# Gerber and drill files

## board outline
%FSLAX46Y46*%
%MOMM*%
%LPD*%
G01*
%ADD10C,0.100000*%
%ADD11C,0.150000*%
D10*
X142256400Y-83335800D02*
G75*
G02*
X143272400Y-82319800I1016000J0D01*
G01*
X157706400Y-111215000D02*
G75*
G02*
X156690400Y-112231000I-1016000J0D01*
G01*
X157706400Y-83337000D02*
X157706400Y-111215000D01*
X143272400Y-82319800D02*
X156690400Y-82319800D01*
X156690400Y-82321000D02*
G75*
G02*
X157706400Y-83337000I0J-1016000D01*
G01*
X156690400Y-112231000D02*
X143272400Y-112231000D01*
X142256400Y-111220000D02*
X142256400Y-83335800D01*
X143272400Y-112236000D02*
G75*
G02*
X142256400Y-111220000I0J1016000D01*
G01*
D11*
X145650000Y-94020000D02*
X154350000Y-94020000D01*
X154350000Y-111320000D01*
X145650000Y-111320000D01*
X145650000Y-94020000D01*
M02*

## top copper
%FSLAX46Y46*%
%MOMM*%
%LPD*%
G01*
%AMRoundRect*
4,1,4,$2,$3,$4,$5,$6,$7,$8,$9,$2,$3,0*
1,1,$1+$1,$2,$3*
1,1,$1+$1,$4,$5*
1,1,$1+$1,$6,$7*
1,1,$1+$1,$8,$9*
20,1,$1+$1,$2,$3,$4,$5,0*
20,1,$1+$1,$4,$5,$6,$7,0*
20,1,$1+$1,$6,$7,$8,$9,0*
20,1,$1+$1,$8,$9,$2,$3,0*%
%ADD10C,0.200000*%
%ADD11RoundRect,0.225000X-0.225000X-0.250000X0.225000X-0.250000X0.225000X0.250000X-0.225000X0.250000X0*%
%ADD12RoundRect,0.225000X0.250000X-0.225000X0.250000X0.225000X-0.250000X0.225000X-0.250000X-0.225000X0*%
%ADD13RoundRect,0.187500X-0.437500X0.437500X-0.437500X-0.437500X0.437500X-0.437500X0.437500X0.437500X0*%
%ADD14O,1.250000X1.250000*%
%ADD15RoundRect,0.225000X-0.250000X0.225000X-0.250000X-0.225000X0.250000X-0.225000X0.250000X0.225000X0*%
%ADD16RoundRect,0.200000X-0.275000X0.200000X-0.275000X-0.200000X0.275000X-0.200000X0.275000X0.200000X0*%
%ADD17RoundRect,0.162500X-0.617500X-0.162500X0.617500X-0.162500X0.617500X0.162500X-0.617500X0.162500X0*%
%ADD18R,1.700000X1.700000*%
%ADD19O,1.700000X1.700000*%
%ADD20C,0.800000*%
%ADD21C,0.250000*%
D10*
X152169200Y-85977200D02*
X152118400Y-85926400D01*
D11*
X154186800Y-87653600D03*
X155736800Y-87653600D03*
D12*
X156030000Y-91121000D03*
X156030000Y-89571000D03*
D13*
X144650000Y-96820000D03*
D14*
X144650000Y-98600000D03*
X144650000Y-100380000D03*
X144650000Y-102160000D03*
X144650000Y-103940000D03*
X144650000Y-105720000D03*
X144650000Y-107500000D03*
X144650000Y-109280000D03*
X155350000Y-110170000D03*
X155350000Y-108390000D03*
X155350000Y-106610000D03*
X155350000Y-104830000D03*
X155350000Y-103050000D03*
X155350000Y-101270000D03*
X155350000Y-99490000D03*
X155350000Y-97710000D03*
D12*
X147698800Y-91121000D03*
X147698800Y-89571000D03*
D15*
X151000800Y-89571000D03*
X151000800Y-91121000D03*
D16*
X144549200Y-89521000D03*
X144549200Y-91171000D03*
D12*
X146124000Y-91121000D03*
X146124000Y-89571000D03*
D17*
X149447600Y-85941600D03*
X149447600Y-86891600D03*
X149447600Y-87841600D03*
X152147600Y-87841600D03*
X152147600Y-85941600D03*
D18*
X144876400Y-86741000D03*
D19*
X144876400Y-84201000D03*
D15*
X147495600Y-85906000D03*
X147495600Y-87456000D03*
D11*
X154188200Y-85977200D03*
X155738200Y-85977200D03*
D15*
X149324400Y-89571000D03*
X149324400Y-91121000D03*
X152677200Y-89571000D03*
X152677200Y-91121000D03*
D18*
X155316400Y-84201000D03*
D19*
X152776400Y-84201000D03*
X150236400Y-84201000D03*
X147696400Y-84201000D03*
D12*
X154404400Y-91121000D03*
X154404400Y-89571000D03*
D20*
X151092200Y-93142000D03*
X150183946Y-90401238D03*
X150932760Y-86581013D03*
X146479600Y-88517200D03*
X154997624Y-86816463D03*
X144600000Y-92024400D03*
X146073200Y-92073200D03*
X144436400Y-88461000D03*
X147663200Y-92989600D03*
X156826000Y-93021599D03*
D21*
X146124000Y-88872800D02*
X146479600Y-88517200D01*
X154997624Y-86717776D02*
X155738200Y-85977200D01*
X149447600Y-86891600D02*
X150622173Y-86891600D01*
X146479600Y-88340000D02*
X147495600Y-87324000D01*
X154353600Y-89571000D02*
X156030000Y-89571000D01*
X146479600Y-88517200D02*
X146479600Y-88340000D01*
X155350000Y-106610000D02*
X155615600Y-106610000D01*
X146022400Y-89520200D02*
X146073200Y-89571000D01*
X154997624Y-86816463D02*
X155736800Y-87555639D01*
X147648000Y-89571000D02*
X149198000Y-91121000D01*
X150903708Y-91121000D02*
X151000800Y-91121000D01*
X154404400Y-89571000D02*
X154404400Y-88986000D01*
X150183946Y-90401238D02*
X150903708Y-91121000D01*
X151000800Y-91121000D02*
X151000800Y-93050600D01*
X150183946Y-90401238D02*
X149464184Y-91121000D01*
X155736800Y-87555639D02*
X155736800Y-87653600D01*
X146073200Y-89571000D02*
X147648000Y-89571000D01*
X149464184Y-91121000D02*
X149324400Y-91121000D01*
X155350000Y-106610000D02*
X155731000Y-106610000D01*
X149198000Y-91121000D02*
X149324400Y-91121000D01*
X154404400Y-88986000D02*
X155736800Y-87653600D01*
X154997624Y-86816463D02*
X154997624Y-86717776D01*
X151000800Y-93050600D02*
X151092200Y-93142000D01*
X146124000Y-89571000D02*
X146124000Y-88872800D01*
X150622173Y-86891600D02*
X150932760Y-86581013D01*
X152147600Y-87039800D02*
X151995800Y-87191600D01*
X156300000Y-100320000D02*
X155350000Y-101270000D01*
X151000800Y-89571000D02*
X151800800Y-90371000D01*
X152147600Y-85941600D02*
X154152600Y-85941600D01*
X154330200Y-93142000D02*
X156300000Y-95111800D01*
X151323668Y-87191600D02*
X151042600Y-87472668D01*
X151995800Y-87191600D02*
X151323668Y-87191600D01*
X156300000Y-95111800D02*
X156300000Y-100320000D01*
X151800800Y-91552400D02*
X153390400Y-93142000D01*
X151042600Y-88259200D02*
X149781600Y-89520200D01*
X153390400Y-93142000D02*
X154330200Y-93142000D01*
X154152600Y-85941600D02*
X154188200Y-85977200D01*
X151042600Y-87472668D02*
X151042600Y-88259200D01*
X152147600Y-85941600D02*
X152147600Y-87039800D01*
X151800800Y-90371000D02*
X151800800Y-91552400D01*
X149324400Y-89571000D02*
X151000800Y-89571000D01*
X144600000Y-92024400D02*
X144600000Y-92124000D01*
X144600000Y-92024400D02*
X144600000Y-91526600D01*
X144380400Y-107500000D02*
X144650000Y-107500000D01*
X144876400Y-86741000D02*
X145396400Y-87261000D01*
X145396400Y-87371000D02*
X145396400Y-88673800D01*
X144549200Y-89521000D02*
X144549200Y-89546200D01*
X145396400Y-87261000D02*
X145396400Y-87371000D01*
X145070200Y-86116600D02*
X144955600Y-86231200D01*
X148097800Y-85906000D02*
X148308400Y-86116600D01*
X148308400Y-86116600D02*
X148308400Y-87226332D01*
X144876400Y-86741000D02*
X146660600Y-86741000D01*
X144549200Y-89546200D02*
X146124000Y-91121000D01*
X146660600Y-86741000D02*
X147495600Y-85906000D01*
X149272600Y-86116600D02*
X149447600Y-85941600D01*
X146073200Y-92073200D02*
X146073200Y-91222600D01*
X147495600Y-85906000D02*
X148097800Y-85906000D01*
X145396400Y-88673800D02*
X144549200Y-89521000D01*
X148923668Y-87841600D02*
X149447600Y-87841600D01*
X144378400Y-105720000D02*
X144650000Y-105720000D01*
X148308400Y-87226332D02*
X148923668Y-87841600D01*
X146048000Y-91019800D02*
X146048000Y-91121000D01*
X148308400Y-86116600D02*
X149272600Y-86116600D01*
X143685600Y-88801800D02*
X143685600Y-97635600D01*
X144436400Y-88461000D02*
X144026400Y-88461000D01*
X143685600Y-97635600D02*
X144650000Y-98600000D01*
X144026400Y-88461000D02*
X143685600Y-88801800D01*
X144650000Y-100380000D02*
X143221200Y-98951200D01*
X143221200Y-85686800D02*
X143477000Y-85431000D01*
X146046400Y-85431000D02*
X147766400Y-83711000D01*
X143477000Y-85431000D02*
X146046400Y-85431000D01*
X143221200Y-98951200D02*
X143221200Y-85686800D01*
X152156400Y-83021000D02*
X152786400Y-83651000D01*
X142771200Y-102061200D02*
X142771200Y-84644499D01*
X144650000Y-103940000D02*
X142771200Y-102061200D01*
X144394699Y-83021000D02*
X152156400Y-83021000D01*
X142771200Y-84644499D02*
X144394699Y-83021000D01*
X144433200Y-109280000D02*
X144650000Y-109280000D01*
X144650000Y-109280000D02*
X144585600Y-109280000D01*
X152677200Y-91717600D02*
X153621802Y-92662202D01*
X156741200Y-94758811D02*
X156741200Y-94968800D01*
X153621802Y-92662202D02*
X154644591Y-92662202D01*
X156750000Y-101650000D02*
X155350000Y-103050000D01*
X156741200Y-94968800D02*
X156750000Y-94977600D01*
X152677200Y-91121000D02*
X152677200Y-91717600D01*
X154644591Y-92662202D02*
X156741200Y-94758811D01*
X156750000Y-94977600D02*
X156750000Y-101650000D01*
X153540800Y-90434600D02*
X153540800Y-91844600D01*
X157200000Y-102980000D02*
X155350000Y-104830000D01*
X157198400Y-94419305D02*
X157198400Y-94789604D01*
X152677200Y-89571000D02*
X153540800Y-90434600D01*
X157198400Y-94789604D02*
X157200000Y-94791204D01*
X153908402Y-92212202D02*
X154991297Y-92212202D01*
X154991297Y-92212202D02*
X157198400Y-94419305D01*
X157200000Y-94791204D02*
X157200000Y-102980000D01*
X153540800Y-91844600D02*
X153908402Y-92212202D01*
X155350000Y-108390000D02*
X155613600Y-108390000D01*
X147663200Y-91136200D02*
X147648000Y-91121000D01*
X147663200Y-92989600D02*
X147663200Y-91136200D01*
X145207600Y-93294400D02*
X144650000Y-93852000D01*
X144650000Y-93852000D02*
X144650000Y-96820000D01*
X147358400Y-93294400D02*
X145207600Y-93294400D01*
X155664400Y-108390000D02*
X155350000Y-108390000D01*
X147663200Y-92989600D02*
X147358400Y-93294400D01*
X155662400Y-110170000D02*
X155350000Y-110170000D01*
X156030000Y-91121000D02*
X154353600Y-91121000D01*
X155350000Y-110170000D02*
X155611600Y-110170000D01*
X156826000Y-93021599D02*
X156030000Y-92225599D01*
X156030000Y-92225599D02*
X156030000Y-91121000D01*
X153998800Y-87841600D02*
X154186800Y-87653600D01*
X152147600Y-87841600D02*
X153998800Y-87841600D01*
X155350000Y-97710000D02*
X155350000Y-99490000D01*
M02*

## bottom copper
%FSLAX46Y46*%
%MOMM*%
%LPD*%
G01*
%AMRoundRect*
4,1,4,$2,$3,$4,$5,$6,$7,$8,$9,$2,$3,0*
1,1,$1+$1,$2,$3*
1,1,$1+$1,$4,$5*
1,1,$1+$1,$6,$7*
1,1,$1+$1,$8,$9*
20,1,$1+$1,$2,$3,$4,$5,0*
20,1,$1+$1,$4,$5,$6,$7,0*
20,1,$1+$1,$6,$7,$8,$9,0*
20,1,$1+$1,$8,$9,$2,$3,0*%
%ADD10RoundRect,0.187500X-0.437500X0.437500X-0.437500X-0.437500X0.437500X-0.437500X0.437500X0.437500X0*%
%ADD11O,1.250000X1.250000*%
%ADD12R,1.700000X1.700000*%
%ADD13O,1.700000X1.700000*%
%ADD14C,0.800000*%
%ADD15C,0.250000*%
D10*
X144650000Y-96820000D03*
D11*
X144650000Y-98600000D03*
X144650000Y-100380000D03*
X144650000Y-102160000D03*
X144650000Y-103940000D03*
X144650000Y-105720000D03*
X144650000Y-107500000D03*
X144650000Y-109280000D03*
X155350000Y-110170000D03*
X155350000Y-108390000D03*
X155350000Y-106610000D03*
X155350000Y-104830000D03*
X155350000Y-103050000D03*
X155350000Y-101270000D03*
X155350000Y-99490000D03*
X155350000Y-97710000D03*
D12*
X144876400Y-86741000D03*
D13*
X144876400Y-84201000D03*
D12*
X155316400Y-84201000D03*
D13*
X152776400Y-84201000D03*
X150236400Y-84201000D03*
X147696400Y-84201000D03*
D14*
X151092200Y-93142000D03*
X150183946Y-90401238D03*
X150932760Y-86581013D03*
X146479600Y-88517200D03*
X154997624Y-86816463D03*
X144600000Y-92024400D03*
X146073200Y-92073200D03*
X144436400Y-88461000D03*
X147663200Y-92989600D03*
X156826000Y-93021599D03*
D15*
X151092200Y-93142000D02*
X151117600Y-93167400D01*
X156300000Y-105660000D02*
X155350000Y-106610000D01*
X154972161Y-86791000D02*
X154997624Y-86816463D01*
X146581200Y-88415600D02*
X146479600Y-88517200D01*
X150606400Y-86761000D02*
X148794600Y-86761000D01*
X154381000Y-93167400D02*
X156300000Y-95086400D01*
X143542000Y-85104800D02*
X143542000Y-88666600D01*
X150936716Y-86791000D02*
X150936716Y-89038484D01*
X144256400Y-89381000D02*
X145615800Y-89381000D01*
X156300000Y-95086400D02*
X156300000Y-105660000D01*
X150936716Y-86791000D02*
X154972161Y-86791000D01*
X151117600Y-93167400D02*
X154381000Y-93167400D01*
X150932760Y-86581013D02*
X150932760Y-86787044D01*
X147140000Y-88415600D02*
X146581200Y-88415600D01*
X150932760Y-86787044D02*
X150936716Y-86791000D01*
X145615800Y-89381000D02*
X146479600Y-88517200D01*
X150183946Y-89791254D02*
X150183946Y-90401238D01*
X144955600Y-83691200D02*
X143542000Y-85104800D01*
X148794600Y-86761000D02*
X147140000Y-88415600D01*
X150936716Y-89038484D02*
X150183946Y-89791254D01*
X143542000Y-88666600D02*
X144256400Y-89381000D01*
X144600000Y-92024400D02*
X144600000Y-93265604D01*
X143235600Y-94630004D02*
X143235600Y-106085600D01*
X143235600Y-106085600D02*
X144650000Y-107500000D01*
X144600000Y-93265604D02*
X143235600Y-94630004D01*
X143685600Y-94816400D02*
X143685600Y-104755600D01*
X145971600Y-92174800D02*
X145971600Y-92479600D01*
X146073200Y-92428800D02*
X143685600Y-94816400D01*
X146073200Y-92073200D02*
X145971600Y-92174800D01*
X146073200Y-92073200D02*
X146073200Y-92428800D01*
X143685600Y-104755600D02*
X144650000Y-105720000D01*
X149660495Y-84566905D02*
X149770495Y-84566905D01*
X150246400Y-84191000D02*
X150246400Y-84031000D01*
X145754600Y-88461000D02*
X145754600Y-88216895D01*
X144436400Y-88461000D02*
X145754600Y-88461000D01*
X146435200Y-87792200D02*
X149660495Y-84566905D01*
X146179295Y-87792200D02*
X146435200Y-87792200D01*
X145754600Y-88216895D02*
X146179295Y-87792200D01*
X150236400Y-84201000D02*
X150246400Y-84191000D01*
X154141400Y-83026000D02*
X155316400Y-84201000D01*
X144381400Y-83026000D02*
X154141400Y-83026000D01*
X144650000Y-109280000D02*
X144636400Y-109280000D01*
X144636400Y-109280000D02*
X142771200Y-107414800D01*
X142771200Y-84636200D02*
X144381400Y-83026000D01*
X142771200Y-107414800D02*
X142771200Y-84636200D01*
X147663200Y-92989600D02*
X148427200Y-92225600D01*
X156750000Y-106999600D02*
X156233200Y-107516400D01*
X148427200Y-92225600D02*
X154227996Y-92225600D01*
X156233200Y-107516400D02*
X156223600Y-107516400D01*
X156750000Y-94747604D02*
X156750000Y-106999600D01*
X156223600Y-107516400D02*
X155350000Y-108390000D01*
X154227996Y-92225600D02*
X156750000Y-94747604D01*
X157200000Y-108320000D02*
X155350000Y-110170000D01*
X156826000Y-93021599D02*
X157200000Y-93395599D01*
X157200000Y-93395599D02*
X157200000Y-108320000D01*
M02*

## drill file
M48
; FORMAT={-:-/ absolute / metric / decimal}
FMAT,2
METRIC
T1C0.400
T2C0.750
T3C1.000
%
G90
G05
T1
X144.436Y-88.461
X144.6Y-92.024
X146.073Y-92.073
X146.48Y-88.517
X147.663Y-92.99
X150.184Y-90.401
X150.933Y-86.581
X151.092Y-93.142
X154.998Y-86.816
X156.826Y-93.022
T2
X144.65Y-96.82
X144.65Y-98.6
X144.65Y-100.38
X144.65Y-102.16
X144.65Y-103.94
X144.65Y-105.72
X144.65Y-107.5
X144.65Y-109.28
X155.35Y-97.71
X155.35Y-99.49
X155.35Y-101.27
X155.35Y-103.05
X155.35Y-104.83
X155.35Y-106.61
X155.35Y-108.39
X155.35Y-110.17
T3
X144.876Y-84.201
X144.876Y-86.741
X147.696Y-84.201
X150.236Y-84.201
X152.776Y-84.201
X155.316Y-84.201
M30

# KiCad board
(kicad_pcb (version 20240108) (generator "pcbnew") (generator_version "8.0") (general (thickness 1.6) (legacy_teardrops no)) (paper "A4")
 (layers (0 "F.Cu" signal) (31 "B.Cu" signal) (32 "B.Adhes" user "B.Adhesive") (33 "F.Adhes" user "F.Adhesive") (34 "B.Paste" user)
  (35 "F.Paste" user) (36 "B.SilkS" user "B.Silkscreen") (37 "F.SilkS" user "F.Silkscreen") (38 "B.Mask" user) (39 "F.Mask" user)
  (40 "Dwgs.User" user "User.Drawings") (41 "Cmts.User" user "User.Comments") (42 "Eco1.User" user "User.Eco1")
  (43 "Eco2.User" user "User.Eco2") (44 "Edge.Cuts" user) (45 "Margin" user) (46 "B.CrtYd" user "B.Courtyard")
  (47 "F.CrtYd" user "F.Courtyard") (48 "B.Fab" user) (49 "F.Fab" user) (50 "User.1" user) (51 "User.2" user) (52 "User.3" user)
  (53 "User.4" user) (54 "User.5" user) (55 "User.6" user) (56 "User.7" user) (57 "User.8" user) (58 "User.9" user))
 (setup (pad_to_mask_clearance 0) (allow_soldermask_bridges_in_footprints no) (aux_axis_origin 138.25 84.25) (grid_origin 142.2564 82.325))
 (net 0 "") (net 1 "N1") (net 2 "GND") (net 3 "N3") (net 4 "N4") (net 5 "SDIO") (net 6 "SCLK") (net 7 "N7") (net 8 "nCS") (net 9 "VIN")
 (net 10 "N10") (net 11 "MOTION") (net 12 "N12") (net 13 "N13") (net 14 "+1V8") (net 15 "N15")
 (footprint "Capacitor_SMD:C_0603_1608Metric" (layer "F.Cu") (at 154.9618 87.6536)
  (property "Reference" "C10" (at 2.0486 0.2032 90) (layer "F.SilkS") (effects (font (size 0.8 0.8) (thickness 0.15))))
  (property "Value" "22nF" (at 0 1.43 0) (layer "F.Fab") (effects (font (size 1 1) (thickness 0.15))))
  (pad "1" smd roundrect (at -0.775 0) (size 0.9 0.95) (layers "F.Cu" "F.Paste" "F.Mask") (roundrect_rratio 0.25) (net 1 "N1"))
  (pad "2" smd roundrect (at 0.775 0) (size 0.9 0.95) (layers "F.Cu" "F.Paste" "F.Mask") (roundrect_rratio 0.25) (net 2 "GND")))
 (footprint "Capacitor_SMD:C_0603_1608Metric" (layer "F.Cu") (at 156.03 90.346 90)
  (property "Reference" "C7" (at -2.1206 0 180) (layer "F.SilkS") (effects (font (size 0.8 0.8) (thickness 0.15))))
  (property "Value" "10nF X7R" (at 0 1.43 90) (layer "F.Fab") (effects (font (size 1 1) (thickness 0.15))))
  (pad "1" smd roundrect (at -0.775 0 90) (size 0.9 0.95) (layers "F.Cu" "F.Paste" "F.Mask") (roundrect_rratio 0.25) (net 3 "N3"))
  (pad "2" smd roundrect (at 0.775 0 90) (size 0.9 0.95) (layers "F.Cu" "F.Paste" "F.Mask") (roundrect_rratio 0.25) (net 2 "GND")))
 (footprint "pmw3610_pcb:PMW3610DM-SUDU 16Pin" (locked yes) (layer "F.Cu") (at 150 102.988 90)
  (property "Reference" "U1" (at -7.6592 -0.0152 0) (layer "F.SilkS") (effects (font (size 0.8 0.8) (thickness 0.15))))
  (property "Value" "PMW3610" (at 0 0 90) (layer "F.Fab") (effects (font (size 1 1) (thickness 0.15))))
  (fp_rect (start 8.968 -4.35) (end -8.332 4.35) (stroke (width 0.15) (type solid)) (fill none) (layer "Edge.Cuts"))
  (pad "1" thru_hole roundrect (at 6.168 -5.35 270) (size 1.25 1.25) (drill 0.75) (layers "*.Cu" "*.Mask") (remove_unused_layers no)
   (roundrect_rratio 0.15) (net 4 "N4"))
  (pad "2" thru_hole oval (at 4.388 -5.35 270) (size 1.25 1.25) (drill 0.75) (layers "*.Cu" "*.Mask") (remove_unused_layers no)
   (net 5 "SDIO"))
  (pad "3" thru_hole oval (at 2.608 -5.35 270) (size 1.25 1.25) (drill 0.75) (layers "*.Cu" "*.Mask") (remove_unused_layers no)
   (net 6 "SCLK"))
  (pad "4" thru_hole oval (at 0.828 -5.35 270) (size 1.25 1.25) (drill 0.75) (layers "*.Cu" "*.Mask") (remove_unused_layers no) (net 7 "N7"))
  (pad "5" thru_hole oval (at -0.952 -5.35 270) (size 1.25 1.25) (drill 0.75) (layers "*.Cu" "*.Mask") (remove_unused_layers no)
   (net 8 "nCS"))
  (pad "6" thru_hole oval (at -2.732 -5.35 270) (size 1.25 1.25) (drill 0.75) (layers "*.Cu" "*.Mask") (remove_unused_layers no)
   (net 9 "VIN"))
  (pad "7" thru_hole oval (at -4.512 -5.35 270) (size 1.25 1.25) (drill 0.75) (layers "*.Cu" "*.Mask") (remove_unused_layers no)
   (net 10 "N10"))
  (pad "8" thru_hole oval (at -6.292 -5.35 270) (size 1.25 1.25) (drill 0.75) (layers "*.Cu" "*.Mask") (remove_unused_layers no)
   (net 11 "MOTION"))
  (pad "9" thru_hole oval (at -7.182 5.35 270) (size 1.25 1.25) (drill 0.75) (layers "*.Cu" "*.Mask") (remove_unused_layers no) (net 3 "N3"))
  (pad "10" thru_hole oval (at -5.402 5.35 270) (size 1.25 1.25) (drill 0.75) (layers "*.Cu" "*.Mask") (remove_unused_layers no)
   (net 4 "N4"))
  (pad "11" thru_hole oval (at -3.622 5.35 270) (size 1.25 1.25) (drill 0.75) (layers "*.Cu" "*.Mask") (remove_unused_layers no)
   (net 2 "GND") (thermal_bridge_angle 45))
  (pad "12" thru_hole oval (at -1.842 5.35 270) (size 1.25 1.25) (drill 0.75) (layers "*.Cu" "*.Mask") (remove_unused_layers no)
   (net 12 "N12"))
  (pad "13" thru_hole oval (at -0.062 5.35 270) (size 1.25 1.25) (drill 0.75) (layers "*.Cu" "*.Mask") (remove_unused_layers no)
   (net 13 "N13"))
  (pad "14" thru_hole oval (at 1.718 5.35 270) (size 1.25 1.25) (drill 0.75) (layers "*.Cu" "*.Mask") (remove_unused_layers no)
   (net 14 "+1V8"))
  (pad "15" thru_hole oval (at 3.498 5.35 270) (size 1.25 1.25) (drill 0.75) (layers "*.Cu" "*.Mask") (remove_unused_layers no)
   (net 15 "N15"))
  (pad "16" thru_hole oval (at 5.278 5.35 270) (size 1.25 1.25) (drill 0.75) (layers "*.Cu" "*.Mask") (remove_unused_layers no)
   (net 15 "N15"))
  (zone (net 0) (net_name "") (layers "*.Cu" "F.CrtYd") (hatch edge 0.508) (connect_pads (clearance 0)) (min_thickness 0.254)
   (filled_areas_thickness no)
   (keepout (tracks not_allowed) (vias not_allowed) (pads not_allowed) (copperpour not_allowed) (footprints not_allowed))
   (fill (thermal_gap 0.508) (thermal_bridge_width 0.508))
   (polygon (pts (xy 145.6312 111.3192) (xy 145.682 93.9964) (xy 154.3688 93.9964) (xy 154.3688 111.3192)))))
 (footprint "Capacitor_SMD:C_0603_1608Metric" (layer "F.Cu") (at 147.6988 90.346 90)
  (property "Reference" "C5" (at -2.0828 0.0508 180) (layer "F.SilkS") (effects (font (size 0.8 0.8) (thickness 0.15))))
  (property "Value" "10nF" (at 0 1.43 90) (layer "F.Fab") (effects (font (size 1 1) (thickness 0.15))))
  (pad "1" smd roundrect (at -0.775 0 90) (size 0.9 0.95) (layers "F.Cu" "F.Paste" "F.Mask") (roundrect_rratio 0.25) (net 4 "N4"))
  (pad "2" smd roundrect (at 0.775 0 90) (size 0.9 0.95) (layers "F.Cu" "F.Paste" "F.Mask") (roundrect_rratio 0.25) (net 2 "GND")))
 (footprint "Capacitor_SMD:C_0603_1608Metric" (layer "F.Cu") (at 151.0008 90.346 -90)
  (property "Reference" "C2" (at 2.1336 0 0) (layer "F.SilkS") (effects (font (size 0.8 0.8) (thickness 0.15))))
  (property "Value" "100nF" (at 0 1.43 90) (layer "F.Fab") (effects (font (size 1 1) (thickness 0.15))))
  (pad "1" smd roundrect (at -0.775 0 270) (size 0.9 0.95) (layers "F.Cu" "F.Paste" "F.Mask") (roundrect_rratio 0.25) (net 14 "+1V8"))
  (pad "2" smd roundrect (at 0.775 0 270) (size 0.9 0.95) (layers "F.Cu" "F.Paste" "F.Mask") (roundrect_rratio 0.25) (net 2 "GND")))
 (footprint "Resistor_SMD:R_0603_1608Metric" (layer "F.Cu") (at 144.5492 90.346 -90)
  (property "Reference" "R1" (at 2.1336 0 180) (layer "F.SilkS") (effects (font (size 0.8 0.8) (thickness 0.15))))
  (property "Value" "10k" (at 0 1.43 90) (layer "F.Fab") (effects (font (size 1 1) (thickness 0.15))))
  (pad "1" smd roundrect (at -0.825 0 270) (size 0.8 0.95) (layers "F.Cu" "F.Paste" "F.Mask") (roundrect_rratio 0.25) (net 9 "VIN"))
  (pad "2" smd roundrect (at 0.825 0 270) (size 0.8 0.95) (layers "F.Cu" "F.Paste" "F.Mask") (roundrect_rratio 0.25) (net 10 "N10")))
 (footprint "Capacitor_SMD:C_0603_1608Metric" (layer "F.Cu") (at 146.124 90.346 90)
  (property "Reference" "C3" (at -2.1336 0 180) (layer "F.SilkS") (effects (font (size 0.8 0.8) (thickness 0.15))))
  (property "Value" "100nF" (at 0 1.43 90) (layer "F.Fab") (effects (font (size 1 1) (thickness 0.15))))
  (pad "1" smd roundrect (at -0.775 0 90) (size 0.9 0.95) (layers "F.Cu" "F.Paste" "F.Mask") (roundrect_rratio 0.25) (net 9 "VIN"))
  (pad "2" smd roundrect (at 0.775 0 90) (size 0.9 0.95) (layers "F.Cu" "F.Paste" "F.Mask") (roundrect_rratio 0.25) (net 2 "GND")))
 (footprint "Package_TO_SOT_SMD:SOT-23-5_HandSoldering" (layer "F.Cu") (at 150.7976 86.8916)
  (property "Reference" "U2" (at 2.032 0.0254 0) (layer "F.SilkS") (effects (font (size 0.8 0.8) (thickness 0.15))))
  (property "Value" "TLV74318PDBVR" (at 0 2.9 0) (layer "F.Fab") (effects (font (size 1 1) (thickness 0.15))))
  (pad "1" smd roundrect (at -1.35 -0.95) (size 1.56 0.65) (layers "F.Cu" "F.Paste" "F.Mask") (roundrect_rratio 0.25) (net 9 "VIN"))
  (pad "2" smd roundrect (at -1.35 0) (size 1.56 0.65) (layers "F.Cu" "F.Paste" "F.Mask") (roundrect_rratio 0.25) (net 2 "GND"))
  (pad "3" smd roundrect (at -1.35 0.95) (size 1.56 0.65) (layers "F.Cu" "F.Paste" "F.Mask") (roundrect_rratio 0.25) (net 9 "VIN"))
  (pad "4" smd roundrect (at 1.35 0.95) (size 1.56 0.65) (layers "F.Cu" "F.Paste" "F.Mask") (roundrect_rratio 0.25) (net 1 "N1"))
  (pad "5" smd roundrect (at 1.35 -0.95) (size 1.56 0.65) (layers "F.Cu" "F.Paste" "F.Mask") (roundrect_rratio 0.25) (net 14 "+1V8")))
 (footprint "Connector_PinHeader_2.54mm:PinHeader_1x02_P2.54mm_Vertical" (layer "F.Cu") (at 144.8764 86.741 180)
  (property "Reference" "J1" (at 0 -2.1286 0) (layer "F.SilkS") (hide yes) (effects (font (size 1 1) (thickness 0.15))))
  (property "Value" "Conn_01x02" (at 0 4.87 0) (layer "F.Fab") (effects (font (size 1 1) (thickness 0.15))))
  (pad "1" thru_hole rect (at 0 0 180) (size 1.7 1.7) (drill 1) (layers "*.Cu" "*.Mask") (remove_unused_layers no) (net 9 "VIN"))
  (pad "2" thru_hole oval (at 0 2.54 180) (size 1.7 1.7) (drill 1) (layers "*.Cu" "*.Mask") (remove_unused_layers no) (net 2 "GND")))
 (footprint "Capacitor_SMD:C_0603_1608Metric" (layer "F.Cu") (at 147.4956 86.681 -90)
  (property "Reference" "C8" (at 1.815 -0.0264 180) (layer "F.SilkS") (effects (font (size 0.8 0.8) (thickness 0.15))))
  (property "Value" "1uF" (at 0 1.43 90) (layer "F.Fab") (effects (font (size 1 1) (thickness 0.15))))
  (pad "1" smd roundrect (at -0.775 0 270) (size 0.9 0.95) (layers "F.Cu" "F.Paste" "F.Mask") (roundrect_rratio 0.25) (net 9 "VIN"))
  (pad "2" smd roundrect (at 0.775 0 270) (size 0.9 0.95) (layers "F.Cu" "F.Paste" "F.Mask") (roundrect_rratio 0.25) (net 2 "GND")))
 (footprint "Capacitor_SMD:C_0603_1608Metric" (layer "F.Cu") (at 154.9632 85.9772)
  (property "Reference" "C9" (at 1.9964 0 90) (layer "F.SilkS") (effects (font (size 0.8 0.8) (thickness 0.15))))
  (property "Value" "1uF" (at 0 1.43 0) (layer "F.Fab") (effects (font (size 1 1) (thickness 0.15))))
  (pad "1" smd roundrect (at -0.775 0) (size 0.9 0.95) (layers "F.Cu" "F.Paste" "F.Mask") (roundrect_rratio 0.25) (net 14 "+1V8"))
  (pad "2" smd roundrect (at 0.775 0) (size 0.9 0.95) (layers "F.Cu" "F.Paste" "F.Mask") (roundrect_rratio 0.25) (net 2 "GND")))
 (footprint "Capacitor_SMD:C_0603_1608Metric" (layer "F.Cu") (at 149.3244 90.346 -90)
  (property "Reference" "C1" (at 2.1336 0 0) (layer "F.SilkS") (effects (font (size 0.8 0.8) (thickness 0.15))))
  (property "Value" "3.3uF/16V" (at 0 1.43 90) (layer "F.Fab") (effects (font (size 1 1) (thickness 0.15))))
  (pad "1" smd roundrect (at -0.775 0 270) (size 0.9 0.95) (layers "F.Cu" "F.Paste" "F.Mask") (roundrect_rratio 0.25) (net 14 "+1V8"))
  (pad "2" smd roundrect (at 0.775 0 270) (size 0.9 0.95) (layers "F.Cu" "F.Paste" "F.Mask") (roundrect_rratio 0.25) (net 2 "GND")))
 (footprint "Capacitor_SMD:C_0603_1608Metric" (layer "F.Cu") (at 152.6772 90.346 -90)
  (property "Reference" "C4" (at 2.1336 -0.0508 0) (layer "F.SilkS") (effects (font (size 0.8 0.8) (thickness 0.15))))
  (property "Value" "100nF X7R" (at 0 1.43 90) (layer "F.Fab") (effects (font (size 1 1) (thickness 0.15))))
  (pad "1" smd roundrect (at -0.775 0 270) (size 0.9 0.95) (layers "F.Cu" "F.Paste" "F.Mask") (roundrect_rratio 0.25) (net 12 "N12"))
  (pad "2" smd roundrect (at 0.775 0 270) (size 0.9 0.95) (layers "F.Cu" "F.Paste" "F.Mask") (roundrect_rratio 0.25) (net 13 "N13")))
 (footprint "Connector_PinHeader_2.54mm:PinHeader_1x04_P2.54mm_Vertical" (layer "F.Cu") (at 155.3164 84.201 -90)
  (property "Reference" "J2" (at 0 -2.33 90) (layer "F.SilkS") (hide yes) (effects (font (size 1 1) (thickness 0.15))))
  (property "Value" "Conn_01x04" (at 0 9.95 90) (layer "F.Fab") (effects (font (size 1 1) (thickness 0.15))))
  (pad "1" thru_hole rect (at 0 0 270) (size 1.7 1.7) (drill 1) (layers "*.Cu" "*.Mask") (remove_unused_layers no) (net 11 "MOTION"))
  (pad "2" thru_hole oval (at 0 2.54 270) (size 1.7 1.7) (drill 1) (layers "*.Cu" "*.Mask") (remove_unused_layers no) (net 8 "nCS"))
  (pad "3" thru_hole oval (at 0 5.08 270) (size 1.7 1.7) (drill 1) (layers "*.Cu" "*.Mask") (remove_unused_layers no) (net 5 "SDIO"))
  (pad "4" thru_hole oval (at 0 7.62 270) (size 1.7 1.7) (drill 1) (layers "*.Cu" "*.Mask") (remove_unused_layers no) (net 6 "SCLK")))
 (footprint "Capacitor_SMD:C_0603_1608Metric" (layer "F.Cu") (at 154.4044 90.346 90)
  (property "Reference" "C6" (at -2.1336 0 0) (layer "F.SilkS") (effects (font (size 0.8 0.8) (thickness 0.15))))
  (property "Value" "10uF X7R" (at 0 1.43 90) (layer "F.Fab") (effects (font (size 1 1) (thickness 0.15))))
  (pad "1" smd roundrect (at -0.775 0 90) (size 0.9 0.95) (layers "F.Cu" "F.Paste" "F.Mask") (roundrect_rratio 0.25) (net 3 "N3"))
  (pad "2" smd roundrect (at 0.775 0 90) (size 0.9 0.95) (layers "F.Cu" "F.Paste" "F.Mask") (roundrect_rratio 0.25) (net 2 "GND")))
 (gr_line (start 152.1692 85.9772) (end 152.1184 85.9264) (stroke (width 0.2) (type default)) (layer "F.Cu") (net 14))
 (gr_arc (start 142.2564 83.3358) (mid 142.55398 82.61738) (end 143.2724 82.3198) (stroke (width 0.1) (type default)) (layer "Edge.Cuts"))
 (gr_arc (start 157.7064 111.215) (mid 157.40882 111.93342) (end 156.6904 112.231) (stroke (width 0.1) (type default)) (layer "Edge.Cuts"))
 (gr_line (start 157.7064 83.337) (end 157.7064 111.215) (stroke (width 0.1) (type default)) (layer "Edge.Cuts"))
 (gr_line (start 143.2724 82.3198) (end 156.6904 82.3198) (stroke (width 0.1) (type default)) (layer "Edge.Cuts"))
 (gr_arc (start 156.6904 82.321) (mid 157.40882 82.61858) (end 157.7064 83.337) (stroke (width 0.1) (type default)) (layer "Edge.Cuts"))
 (gr_line (start 156.6904 112.231) (end 143.2724 112.231) (stroke (width 0.1) (type default)) (layer "Edge.Cuts"))
 (gr_line (start 142.2564 111.22) (end 142.2564 83.3358) (stroke (width 0.1) (type default)) (layer "Edge.Cuts"))
 (gr_arc (start 143.2724 112.236) (mid 142.55398 111.93842) (end 142.2564 111.22) (stroke (width 0.1) (type default)) (layer "Edge.Cuts"))
 (segment (start 146.124 88.8728) (end 146.4796 88.5172) (width 0.25) (layer "F.Cu") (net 2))
 (segment (start 154.997624 86.717776) (end 155.7382 85.9772) (width 0.25) (layer "F.Cu") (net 2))
 (segment (start 149.4476 86.8916) (end 150.622173 86.8916) (width 0.25) (layer "F.Cu") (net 2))
 (segment (start 146.4796 88.34) (end 147.4956 87.324) (width 0.25) (layer "F.Cu") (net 2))
 (segment (start 154.3536 89.571) (end 156.03 89.571) (width 0.25) (layer "F.Cu") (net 2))
 (segment (start 146.4796 88.5172) (end 146.4796 88.34) (width 0.25) (layer "F.Cu") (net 2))
 (segment (start 155.35 106.61) (end 155.6156 106.61) (width 0.25) (layer "F.Cu") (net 2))
 (segment (start 146.0224 89.5202) (end 146.0732 89.571) (width 0.25) (layer "F.Cu") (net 2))
 (segment (start 154.997624 86.816463) (end 155.7368 87.555639) (width 0.25) (layer "F.Cu") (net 2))
 (segment (start 147.648 89.571) (end 149.198 91.121) (width 0.25) (layer "F.Cu") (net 2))
 (segment (start 150.903708 91.121) (end 151.0008 91.121) (width 0.25) (layer "F.Cu") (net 2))
 (segment (start 154.4044 89.571) (end 154.4044 88.986) (width 0.25) (layer "F.Cu") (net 2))
 (segment (start 150.183946 90.401238) (end 150.903708 91.121) (width 0.25) (layer "F.Cu") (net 2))
 (segment (start 151.0008 91.121) (end 151.0008 93.0506) (width 0.25) (layer "F.Cu") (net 2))
 (segment (start 150.183946 90.401238) (end 149.464184 91.121) (width 0.25) (layer "F.Cu") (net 2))
 (segment (start 155.7368 87.555639) (end 155.7368 87.6536) (width 0.25) (layer "F.Cu") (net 2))
 (segment (start 146.0732 89.571) (end 147.648 89.571) (width 0.25) (layer "F.Cu") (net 2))
 (segment (start 149.464184 91.121) (end 149.3244 91.121) (width 0.25) (layer "F.Cu") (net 2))
 (segment (start 155.35 106.61) (end 155.731 106.61) (width 0.25) (layer "F.Cu") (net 2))
 (segment (start 149.198 91.121) (end 149.3244 91.121) (width 0.25) (layer "F.Cu") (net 2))
 (segment (start 154.4044 88.986) (end 155.7368 87.6536) (width 0.25) (layer "F.Cu") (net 2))
 (segment (start 154.997624 86.816463) (end 154.997624 86.717776) (width 0.25) (layer "F.Cu") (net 2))
 (segment (start 151.0008 93.0506) (end 151.0922 93.142) (width 0.25) (layer "F.Cu") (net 2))
 (segment (start 146.124 89.571) (end 146.124 88.8728) (width 0.25) (layer "F.Cu") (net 2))
 (segment (start 150.622173 86.8916) (end 150.93276 86.581013) (width 0.25) (layer "F.Cu") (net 2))
 (via (at 151.0922 93.142) (size 0.8) (drill 0.4) (layers "F.Cu" "B.Cu") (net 2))
 (via (at 150.183946 90.401238) (size 0.8) (drill 0.4) (layers "F.Cu" "B.Cu") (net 2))
 (via (at 150.93276 86.581013) (size 0.8) (drill 0.4) (layers "F.Cu" "B.Cu") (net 2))
 (via (at 146.4796 88.5172) (size 0.8) (drill 0.4) (layers "F.Cu" "B.Cu") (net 2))
 (via (at 154.997624 86.816463) (size 0.8) (drill 0.4) (layers "F.Cu" "B.Cu") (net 2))
 (segment (start 151.0922 93.142) (end 151.1176 93.1674) (width 0.25) (layer "B.Cu") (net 2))
 (segment (start 156.3 105.66) (end 155.35 106.61) (width 0.25) (layer "B.Cu") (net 2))
 (segment (start 154.972161 86.791) (end 154.997624 86.816463) (width 0.25) (layer "B.Cu") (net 2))
 (segment (start 146.5812 88.4156) (end 146.4796 88.5172) (width 0.25) (layer "B.Cu") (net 2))
 (segment (start 150.6064 86.761) (end 148.7946 86.761) (width 0.25) (layer "B.Cu") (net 2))
 (segment (start 154.381 93.1674) (end 156.3 95.0864) (width 0.25) (layer "B.Cu") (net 2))
 (segment (start 143.542 85.1048) (end 143.542 88.6666) (width 0.25) (layer "B.Cu") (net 2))
 (segment (start 150.936716 86.791) (end 150.936716 89.038484) (width 0.25) (layer "B.Cu") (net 2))
 (segment (start 144.2564 89.381) (end 145.6158 89.381) (width 0.25) (layer "B.Cu") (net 2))
 (segment (start 156.3 95.0864) (end 156.3 105.66) (width 0.25) (layer "B.Cu") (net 2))
 (segment (start 150.936716 86.791) (end 154.972161 86.791) (width 0.25) (layer "B.Cu") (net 2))
 (segment (start 151.1176 93.1674) (end 154.381 93.1674) (width 0.25) (layer "B.Cu") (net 2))
 (segment (start 150.93276 86.581013) (end 150.93276 86.787044) (width 0.25) (layer "B.Cu") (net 2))
 (segment (start 147.14 88.4156) (end 146.5812 88.4156) (width 0.25) (layer "B.Cu") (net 2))
 (segment (start 150.93276 86.787044) (end 150.936716 86.791) (width 0.25) (layer "B.Cu") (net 2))
 (segment (start 145.6158 89.381) (end 146.4796 88.5172) (width 0.25) (layer "B.Cu") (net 2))
 (segment (start 150.183946 89.791254) (end 150.183946 90.401238) (width 0.25) (layer "B.Cu") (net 2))
 (segment (start 144.9556 83.6912) (end 143.542 85.1048) (width 0.25) (layer "B.Cu") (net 2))
 (segment (start 148.7946 86.761) (end 147.14 88.4156) (width 0.25) (layer "B.Cu") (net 2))
 (segment (start 150.936716 89.038484) (end 150.183946 89.791254) (width 0.25) (layer "B.Cu") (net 2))
 (segment (start 143.542 88.6666) (end 144.2564 89.381) (width 0.25) (layer "B.Cu") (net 2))
 (segment (start 152.1476 87.0398) (end 151.9958 87.1916) (width 0.25) (layer "F.Cu") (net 14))
 (segment (start 156.3 100.32) (end 155.35 101.27) (width 0.25) (layer "F.Cu") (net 14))
 (segment (start 151.0008 89.571) (end 151.8008 90.371) (width 0.25) (layer "F.Cu") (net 14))
 (segment (start 152.1476 85.9416) (end 154.1526 85.9416) (width 0.25) (layer "F.Cu") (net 14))
 (segment (start 154.3302 93.142) (end 156.3 95.1118) (width 0.25) (layer "F.Cu") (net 14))
 (segment (start 151.323668 87.1916) (end 151.0426 87.472668) (width 0.25) (layer "F.Cu") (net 14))
 (segment (start 151.9958 87.1916) (end 151.323668 87.1916) (width 0.25) (layer "F.Cu") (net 14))
 (segment (start 156.3 95.1118) (end 156.3 100.32) (width 0.25) (layer "F.Cu") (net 14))
 (segment (start 151.8008 91.5524) (end 153.3904 93.142) (width 0.25) (layer "F.Cu") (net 14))
 (segment (start 151.0426 88.2592) (end 149.7816 89.5202) (width 0.25) (layer "F.Cu") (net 14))
 (segment (start 153.3904 93.142) (end 154.3302 93.142) (width 0.25) (layer "F.Cu") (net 14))
 (segment (start 154.1526 85.9416) (end 154.1882 85.9772) (width 0.25) (layer "F.Cu") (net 14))
 (segment (start 151.0426 87.472668) (end 151.0426 88.2592) (width 0.25) (layer "F.Cu") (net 14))
 (segment (start 152.1476 85.9416) (end 152.1476 87.0398) (width 0.25) (layer "F.Cu") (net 14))
 (segment (start 151.8008 90.371) (end 151.8008 91.5524) (width 0.25) (layer "F.Cu") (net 14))
 (segment (start 149.3244 89.571) (end 151.0008 89.571) (width 0.25) (layer "F.Cu") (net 14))
 (segment (start 144.6 92.0244) (end 144.6 92.124) (width 0.25) (layer "F.Cu") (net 10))
 (segment (start 144.6 92.0244) (end 144.6 91.5266) (width 0.25) (layer "F.Cu") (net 10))
 (segment (start 144.3804 107.5) (end 144.65 107.5) (width 0.25) (layer "F.Cu") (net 10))
 (via (at 144.6 92.0244) (size 0.8) (drill 0.4) (layers "F.Cu" "B.Cu") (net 10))
 (segment (start 144.6 92.0244) (end 144.6 93.265604) (width 0.25) (layer "B.Cu") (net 10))
 (segment (start 143.2356 94.630004) (end 143.2356 106.0856) (width 0.25) (layer "B.Cu") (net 10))
 (segment (start 143.2356 106.0856) (end 144.65 107.5) (width 0.25) (layer "B.Cu") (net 10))
 (segment (start 144.6 93.265604) (end 143.2356 94.630004) (width 0.25) (layer "B.Cu") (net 10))
 (segment (start 144.8764 86.741) (end 145.3964 87.261) (width 0.25) (layer "F.Cu") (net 9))
 (segment (start 145.3964 87.371) (end 145.3964 88.6738) (width 0.25) (layer "F.Cu") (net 9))
 (segment (start 144.5492 89.521) (end 144.5492 89.5462) (width 0.25) (layer "F.Cu") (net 9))
 (segment (start 145.3964 87.261) (end 145.3964 87.371) (width 0.25) (layer "F.Cu") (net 9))
 (segment (start 145.0702 86.1166) (end 144.9556 86.2312) (width 0.25) (layer "F.Cu") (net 9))
 (segment (start 148.0978 85.906) (end 148.3084 86.1166) (width 0.25) (layer "F.Cu") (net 9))
 (segment (start 148.3084 86.1166) (end 148.3084 87.226332) (width 0.25) (layer "F.Cu") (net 9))
 (segment (start 144.8764 86.741) (end 146.6606 86.741) (width 0.25) (layer "F.Cu") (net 9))
 (segment (start 144.5492 89.5462) (end 146.124 91.121) (width 0.25) (layer "F.Cu") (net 9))
 (segment (start 146.6606 86.741) (end 147.4956 85.906) (width 0.25) (layer "F.Cu") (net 9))
 (segment (start 149.2726 86.1166) (end 149.4476 85.9416) (width 0.25) (layer "F.Cu") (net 9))
 (segment (start 146.0732 92.0732) (end 146.0732 91.2226) (width 0.25) (layer "F.Cu") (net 9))
 (segment (start 147.4956 85.906) (end 148.0978 85.906) (width 0.25) (layer "F.Cu") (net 9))
 (segment (start 145.3964 88.6738) (end 144.5492 89.521) (width 0.25) (layer "F.Cu") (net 9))
 (segment (start 148.923668 87.8416) (end 149.4476 87.8416) (width 0.25) (layer "F.Cu") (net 9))
 (segment (start 144.3784 105.72) (end 144.65 105.72) (width 0.25) (layer "F.Cu") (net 9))
 (segment (start 148.3084 87.226332) (end 148.923668 87.8416) (width 0.25) (layer "F.Cu") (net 9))
 (segment (start 146.048 91.0198) (end 146.048 91.121) (width 0.25) (layer "F.Cu") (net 9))
 (segment (start 148.3084 86.1166) (end 149.2726 86.1166) (width 0.25) (layer "F.Cu") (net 9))
 (via (at 146.0732 92.0732) (size 0.8) (drill 0.4) (layers "F.Cu" "B.Cu") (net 9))
 (segment (start 143.6856 94.8164) (end 143.6856 104.7556) (width 0.25) (layer "B.Cu") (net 9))
 (segment (start 145.9716 92.1748) (end 145.9716 92.4796) (width 0.25) (layer "B.Cu") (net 9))
 (segment (start 146.0732 92.4288) (end 143.6856 94.8164) (width 0.25) (layer "B.Cu") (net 9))
 (segment (start 146.0732 92.0732) (end 145.9716 92.1748) (width 0.25) (layer "B.Cu") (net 9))
 (segment (start 146.0732 92.0732) (end 146.0732 92.4288) (width 0.25) (layer "B.Cu") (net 9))
 (segment (start 143.6856 104.7556) (end 144.65 105.72) (width 0.25) (layer "B.Cu") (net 9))
 (segment (start 143.6856 88.8018) (end 143.6856 97.6356) (width 0.25) (layer "F.Cu") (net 5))
 (segment (start 144.4364 88.461) (end 144.0264 88.461) (width 0.25) (layer "F.Cu") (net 5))
 (segment (start 143.6856 97.6356) (end 144.65 98.6) (width 0.25) (layer "F.Cu") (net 5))
 (segment (start 144.0264 88.461) (end 143.6856 88.8018) (width 0.25) (layer "F.Cu") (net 5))
 (via (at 144.4364 88.461) (size 0.8) (drill 0.4) (layers "F.Cu" "B.Cu") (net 5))
 (segment (start 149.660495 84.566905) (end 149.770495 84.566905) (width 0.25) (layer "B.Cu") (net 5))
 (segment (start 150.2464 84.191) (end 150.2464 84.031) (width 0.25) (layer "B.Cu") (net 5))
 (segment (start 145.7546 88.461) (end 145.7546 88.216895) (width 0.25) (layer "B.Cu") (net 5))
 (segment (start 144.4364 88.461) (end 145.7546 88.461) (width 0.25) (layer "B.Cu") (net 5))
 (segment (start 146.4352 87.7922) (end 149.660495 84.566905) (width 0.25) (layer "B.Cu") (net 5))
 (segment (start 146.179295 87.7922) (end 146.4352 87.7922) (width 0.25) (layer "B.Cu") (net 5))
 (segment (start 145.7546 88.216895) (end 146.179295 87.7922) (width 0.25) (layer "B.Cu") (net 5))
 (segment (start 150.2364 84.201) (end 150.2464 84.191) (width 0.25) (layer "B.Cu") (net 5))
 (segment (start 144.65 100.38) (end 143.2212 98.9512) (width 0.25) (layer "F.Cu") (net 6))
 (segment (start 143.2212 85.6868) (end 143.477 85.431) (width 0.25) (layer "F.Cu") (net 6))
 (segment (start 146.0464 85.431) (end 147.7664 83.711) (width 0.25) (layer "F.Cu") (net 6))
 (segment (start 143.477 85.431) (end 146.0464 85.431) (width 0.25) (layer "F.Cu") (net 6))
 (segment (start 143.2212 98.9512) (end 143.2212 85.6868) (width 0.25) (layer "F.Cu") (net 6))
 (segment (start 152.1564 83.021) (end 152.7864 83.651) (width 0.25) (layer "F.Cu") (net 8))
 (segment (start 142.7712 102.0612) (end 142.7712 84.644499) (width 0.25) (layer "F.Cu") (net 8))
 (segment (start 144.65 103.94) (end 142.7712 102.0612) (width 0.25) (layer "F.Cu") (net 8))
 (segment (start 144.394699 83.021) (end 152.1564 83.021) (width 0.25) (layer "F.Cu") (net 8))
 (segment (start 142.7712 84.644499) (end 144.394699 83.021) (width 0.25) (layer "F.Cu") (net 8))
 (segment (start 144.4332 109.28) (end 144.65 109.28) (width 0.25) (layer "F.Cu") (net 11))
 (segment (start 144.65 109.28) (end 144.5856 109.28) (width 0.25) (layer "F.Cu") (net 11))
 (segment (start 154.1414 83.026) (end 155.3164 84.201) (width 0.25) (layer "B.Cu") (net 11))
 (segment (start 144.3814 83.026) (end 154.1414 83.026) (width 0.25) (layer "B.Cu") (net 11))
 (segment (start 144.65 109.28) (end 144.6364 109.28) (width 0.25) (layer "B.Cu") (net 11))
 (segment (start 144.6364 109.28) (end 142.7712 107.4148) (width 0.25) (layer "B.Cu") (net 11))
 (segment (start 142.7712 84.6362) (end 144.3814 83.026) (width 0.25) (layer "B.Cu") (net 11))
 (segment (start 142.7712 107.4148) (end 142.7712 84.6362) (width 0.25) (layer "B.Cu") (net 11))
 (segment (start 152.6772 91.7176) (end 153.621802 92.662202) (width 0.25) (layer "F.Cu") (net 13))
 (segment (start 156.7412 94.758811) (end 156.7412 94.9688) (width 0.25) (layer "F.Cu") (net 13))
 (segment (start 153.621802 92.662202) (end 154.644591 92.662202) (width 0.25) (layer "F.Cu") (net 13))
 (segment (start 156.75 101.65) (end 155.35 103.05) (width 0.25) (layer "F.Cu") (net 13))
 (segment (start 156.7412 94.9688) (end 156.75 94.9776) (width 0.25) (layer "F.Cu") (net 13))
 (segment (start 152.6772 91.121) (end 152.6772 91.7176) (width 0.25) (layer "F.Cu") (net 13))
 (segment (start 154.644591 92.662202) (end 156.7412 94.758811) (width 0.25) (layer "F.Cu") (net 13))
 (segment (start 156.75 94.9776) (end 156.75 101.65) (width 0.25) (layer "F.Cu") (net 13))
 (segment (start 153.5408 90.4346) (end 153.5408 91.8446) (width 0.25) (layer "F.Cu") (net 12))
 (segment (start 157.2 102.98) (end 155.35 104.83) (width 0.25) (layer "F.Cu") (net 12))
 (segment (start 157.1984 94.419305) (end 157.1984 94.789604) (width 0.25) (layer "F.Cu") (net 12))
 (segment (start 152.6772 89.571) (end 153.5408 90.4346) (width 0.25) (layer "F.Cu") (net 12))
 (segment (start 157.1984 94.789604) (end 157.2 94.791204) (width 0.25) (layer "F.Cu") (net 12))
 (segment (start 153.908402 92.212202) (end 154.991297 92.212202) (width 0.25) (layer "F.Cu") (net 12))
 (segment (start 154.991297 92.212202) (end 157.1984 94.419305) (width 0.25) (layer "F.Cu") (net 12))
 (segment (start 157.2 94.791204) (end 157.2 102.98) (width 0.25) (layer "F.Cu") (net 12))
 (segment (start 153.5408 91.8446) (end 153.908402 92.212202) (width 0.25) (layer "F.Cu") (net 12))
 (segment (start 155.35 108.39) (end 155.6136 108.39) (width 0.25) (layer "F.Cu") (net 4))
 (segment (start 147.6632 91.1362) (end 147.648 91.121) (width 0.25) (layer "F.Cu") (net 4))
 (segment (start 147.6632 92.9896) (end 147.6632 91.1362) (width 0.25) (layer "F.Cu") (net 4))
 (segment (start 145.2076 93.2944) (end 144.65 93.852) (width 0.25) (layer "F.Cu") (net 4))
 (segment (start 144.65 93.852) (end 144.65 96.82) (width 0.25) (layer "F.Cu") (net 4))
 (segment (start 147.3584 93.2944) (end 145.2076 93.2944) (width 0.25) (layer "F.Cu") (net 4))
 (segment (start 155.6644 108.39) (end 155.35 108.39) (width 0.25) (layer "F.Cu") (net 4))
 (segment (start 147.6632 92.9896) (end 147.3584 93.2944) (width 0.25) (layer "F.Cu") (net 4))
 (via (at 147.6632 92.9896) (size 0.8) (drill 0.4) (layers "F.Cu" "B.Cu") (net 4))
 (segment (start 147.6632 92.9896) (end 148.4272 92.2256) (width 0.25) (layer "B.Cu") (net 4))
 (segment (start 156.75 106.9996) (end 156.2332 107.5164) (width 0.25) (layer "B.Cu") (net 4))
 (segment (start 148.4272 92.2256) (end 154.227996 92.2256) (width 0.25) (layer "B.Cu") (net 4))
 (segment (start 156.2332 107.5164) (end 156.2236 107.5164) (width 0.25) (layer "B.Cu") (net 4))
 (segment (start 156.75 94.747604) (end 156.75 106.9996) (width 0.25) (layer "B.Cu") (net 4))
 (segment (start 156.2236 107.5164) (end 155.35 108.39) (width 0.25) (layer "B.Cu") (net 4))
 (segment (start 154.227996 92.2256) (end 156.75 94.747604) (width 0.25) (layer "B.Cu") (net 4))
 (segment (start 155.6624 110.17) (end 155.35 110.17) (width 0.25) (layer "F.Cu") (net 3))
 (segment (start 156.03 91.121) (end 154.3536 91.121) (width 0.25) (layer "F.Cu") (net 3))
 (segment (start 155.35 110.17) (end 155.6116 110.17) (width 0.25) (layer "F.Cu") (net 3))
 (segment (start 156.826 93.021599) (end 156.03 92.225599) (width 0.25) (layer "F.Cu") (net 3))
 (segment (start 156.03 92.225599) (end 156.03 91.121) (width 0.25) (layer "F.Cu") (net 3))
 (via (at 156.826 93.021599) (size 0.8) (drill 0.4) (layers "F.Cu" "B.Cu") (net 3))
 (segment (start 157.2 108.32) (end 155.35 110.17) (width 0.25) (layer "B.Cu") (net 3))
 (segment (start 156.826 93.021599) (end 157.2 93.395599) (width 0.25) (layer "B.Cu") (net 3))
 (segment (start 157.2 93.395599) (end 157.2 108.32) (width 0.25) (layer "B.Cu") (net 3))
 (segment (start 153.9988 87.8416) (end 154.1868 87.6536) (width 0.25) (layer "F.Cu") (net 1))
 (segment (start 152.1476 87.8416) (end 153.9988 87.8416) (width 0.25) (layer "F.Cu") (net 1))
 (segment (start 155.35 97.71) (end 155.35 99.49) (width 0.25) (layer "F.Cu") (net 15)))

